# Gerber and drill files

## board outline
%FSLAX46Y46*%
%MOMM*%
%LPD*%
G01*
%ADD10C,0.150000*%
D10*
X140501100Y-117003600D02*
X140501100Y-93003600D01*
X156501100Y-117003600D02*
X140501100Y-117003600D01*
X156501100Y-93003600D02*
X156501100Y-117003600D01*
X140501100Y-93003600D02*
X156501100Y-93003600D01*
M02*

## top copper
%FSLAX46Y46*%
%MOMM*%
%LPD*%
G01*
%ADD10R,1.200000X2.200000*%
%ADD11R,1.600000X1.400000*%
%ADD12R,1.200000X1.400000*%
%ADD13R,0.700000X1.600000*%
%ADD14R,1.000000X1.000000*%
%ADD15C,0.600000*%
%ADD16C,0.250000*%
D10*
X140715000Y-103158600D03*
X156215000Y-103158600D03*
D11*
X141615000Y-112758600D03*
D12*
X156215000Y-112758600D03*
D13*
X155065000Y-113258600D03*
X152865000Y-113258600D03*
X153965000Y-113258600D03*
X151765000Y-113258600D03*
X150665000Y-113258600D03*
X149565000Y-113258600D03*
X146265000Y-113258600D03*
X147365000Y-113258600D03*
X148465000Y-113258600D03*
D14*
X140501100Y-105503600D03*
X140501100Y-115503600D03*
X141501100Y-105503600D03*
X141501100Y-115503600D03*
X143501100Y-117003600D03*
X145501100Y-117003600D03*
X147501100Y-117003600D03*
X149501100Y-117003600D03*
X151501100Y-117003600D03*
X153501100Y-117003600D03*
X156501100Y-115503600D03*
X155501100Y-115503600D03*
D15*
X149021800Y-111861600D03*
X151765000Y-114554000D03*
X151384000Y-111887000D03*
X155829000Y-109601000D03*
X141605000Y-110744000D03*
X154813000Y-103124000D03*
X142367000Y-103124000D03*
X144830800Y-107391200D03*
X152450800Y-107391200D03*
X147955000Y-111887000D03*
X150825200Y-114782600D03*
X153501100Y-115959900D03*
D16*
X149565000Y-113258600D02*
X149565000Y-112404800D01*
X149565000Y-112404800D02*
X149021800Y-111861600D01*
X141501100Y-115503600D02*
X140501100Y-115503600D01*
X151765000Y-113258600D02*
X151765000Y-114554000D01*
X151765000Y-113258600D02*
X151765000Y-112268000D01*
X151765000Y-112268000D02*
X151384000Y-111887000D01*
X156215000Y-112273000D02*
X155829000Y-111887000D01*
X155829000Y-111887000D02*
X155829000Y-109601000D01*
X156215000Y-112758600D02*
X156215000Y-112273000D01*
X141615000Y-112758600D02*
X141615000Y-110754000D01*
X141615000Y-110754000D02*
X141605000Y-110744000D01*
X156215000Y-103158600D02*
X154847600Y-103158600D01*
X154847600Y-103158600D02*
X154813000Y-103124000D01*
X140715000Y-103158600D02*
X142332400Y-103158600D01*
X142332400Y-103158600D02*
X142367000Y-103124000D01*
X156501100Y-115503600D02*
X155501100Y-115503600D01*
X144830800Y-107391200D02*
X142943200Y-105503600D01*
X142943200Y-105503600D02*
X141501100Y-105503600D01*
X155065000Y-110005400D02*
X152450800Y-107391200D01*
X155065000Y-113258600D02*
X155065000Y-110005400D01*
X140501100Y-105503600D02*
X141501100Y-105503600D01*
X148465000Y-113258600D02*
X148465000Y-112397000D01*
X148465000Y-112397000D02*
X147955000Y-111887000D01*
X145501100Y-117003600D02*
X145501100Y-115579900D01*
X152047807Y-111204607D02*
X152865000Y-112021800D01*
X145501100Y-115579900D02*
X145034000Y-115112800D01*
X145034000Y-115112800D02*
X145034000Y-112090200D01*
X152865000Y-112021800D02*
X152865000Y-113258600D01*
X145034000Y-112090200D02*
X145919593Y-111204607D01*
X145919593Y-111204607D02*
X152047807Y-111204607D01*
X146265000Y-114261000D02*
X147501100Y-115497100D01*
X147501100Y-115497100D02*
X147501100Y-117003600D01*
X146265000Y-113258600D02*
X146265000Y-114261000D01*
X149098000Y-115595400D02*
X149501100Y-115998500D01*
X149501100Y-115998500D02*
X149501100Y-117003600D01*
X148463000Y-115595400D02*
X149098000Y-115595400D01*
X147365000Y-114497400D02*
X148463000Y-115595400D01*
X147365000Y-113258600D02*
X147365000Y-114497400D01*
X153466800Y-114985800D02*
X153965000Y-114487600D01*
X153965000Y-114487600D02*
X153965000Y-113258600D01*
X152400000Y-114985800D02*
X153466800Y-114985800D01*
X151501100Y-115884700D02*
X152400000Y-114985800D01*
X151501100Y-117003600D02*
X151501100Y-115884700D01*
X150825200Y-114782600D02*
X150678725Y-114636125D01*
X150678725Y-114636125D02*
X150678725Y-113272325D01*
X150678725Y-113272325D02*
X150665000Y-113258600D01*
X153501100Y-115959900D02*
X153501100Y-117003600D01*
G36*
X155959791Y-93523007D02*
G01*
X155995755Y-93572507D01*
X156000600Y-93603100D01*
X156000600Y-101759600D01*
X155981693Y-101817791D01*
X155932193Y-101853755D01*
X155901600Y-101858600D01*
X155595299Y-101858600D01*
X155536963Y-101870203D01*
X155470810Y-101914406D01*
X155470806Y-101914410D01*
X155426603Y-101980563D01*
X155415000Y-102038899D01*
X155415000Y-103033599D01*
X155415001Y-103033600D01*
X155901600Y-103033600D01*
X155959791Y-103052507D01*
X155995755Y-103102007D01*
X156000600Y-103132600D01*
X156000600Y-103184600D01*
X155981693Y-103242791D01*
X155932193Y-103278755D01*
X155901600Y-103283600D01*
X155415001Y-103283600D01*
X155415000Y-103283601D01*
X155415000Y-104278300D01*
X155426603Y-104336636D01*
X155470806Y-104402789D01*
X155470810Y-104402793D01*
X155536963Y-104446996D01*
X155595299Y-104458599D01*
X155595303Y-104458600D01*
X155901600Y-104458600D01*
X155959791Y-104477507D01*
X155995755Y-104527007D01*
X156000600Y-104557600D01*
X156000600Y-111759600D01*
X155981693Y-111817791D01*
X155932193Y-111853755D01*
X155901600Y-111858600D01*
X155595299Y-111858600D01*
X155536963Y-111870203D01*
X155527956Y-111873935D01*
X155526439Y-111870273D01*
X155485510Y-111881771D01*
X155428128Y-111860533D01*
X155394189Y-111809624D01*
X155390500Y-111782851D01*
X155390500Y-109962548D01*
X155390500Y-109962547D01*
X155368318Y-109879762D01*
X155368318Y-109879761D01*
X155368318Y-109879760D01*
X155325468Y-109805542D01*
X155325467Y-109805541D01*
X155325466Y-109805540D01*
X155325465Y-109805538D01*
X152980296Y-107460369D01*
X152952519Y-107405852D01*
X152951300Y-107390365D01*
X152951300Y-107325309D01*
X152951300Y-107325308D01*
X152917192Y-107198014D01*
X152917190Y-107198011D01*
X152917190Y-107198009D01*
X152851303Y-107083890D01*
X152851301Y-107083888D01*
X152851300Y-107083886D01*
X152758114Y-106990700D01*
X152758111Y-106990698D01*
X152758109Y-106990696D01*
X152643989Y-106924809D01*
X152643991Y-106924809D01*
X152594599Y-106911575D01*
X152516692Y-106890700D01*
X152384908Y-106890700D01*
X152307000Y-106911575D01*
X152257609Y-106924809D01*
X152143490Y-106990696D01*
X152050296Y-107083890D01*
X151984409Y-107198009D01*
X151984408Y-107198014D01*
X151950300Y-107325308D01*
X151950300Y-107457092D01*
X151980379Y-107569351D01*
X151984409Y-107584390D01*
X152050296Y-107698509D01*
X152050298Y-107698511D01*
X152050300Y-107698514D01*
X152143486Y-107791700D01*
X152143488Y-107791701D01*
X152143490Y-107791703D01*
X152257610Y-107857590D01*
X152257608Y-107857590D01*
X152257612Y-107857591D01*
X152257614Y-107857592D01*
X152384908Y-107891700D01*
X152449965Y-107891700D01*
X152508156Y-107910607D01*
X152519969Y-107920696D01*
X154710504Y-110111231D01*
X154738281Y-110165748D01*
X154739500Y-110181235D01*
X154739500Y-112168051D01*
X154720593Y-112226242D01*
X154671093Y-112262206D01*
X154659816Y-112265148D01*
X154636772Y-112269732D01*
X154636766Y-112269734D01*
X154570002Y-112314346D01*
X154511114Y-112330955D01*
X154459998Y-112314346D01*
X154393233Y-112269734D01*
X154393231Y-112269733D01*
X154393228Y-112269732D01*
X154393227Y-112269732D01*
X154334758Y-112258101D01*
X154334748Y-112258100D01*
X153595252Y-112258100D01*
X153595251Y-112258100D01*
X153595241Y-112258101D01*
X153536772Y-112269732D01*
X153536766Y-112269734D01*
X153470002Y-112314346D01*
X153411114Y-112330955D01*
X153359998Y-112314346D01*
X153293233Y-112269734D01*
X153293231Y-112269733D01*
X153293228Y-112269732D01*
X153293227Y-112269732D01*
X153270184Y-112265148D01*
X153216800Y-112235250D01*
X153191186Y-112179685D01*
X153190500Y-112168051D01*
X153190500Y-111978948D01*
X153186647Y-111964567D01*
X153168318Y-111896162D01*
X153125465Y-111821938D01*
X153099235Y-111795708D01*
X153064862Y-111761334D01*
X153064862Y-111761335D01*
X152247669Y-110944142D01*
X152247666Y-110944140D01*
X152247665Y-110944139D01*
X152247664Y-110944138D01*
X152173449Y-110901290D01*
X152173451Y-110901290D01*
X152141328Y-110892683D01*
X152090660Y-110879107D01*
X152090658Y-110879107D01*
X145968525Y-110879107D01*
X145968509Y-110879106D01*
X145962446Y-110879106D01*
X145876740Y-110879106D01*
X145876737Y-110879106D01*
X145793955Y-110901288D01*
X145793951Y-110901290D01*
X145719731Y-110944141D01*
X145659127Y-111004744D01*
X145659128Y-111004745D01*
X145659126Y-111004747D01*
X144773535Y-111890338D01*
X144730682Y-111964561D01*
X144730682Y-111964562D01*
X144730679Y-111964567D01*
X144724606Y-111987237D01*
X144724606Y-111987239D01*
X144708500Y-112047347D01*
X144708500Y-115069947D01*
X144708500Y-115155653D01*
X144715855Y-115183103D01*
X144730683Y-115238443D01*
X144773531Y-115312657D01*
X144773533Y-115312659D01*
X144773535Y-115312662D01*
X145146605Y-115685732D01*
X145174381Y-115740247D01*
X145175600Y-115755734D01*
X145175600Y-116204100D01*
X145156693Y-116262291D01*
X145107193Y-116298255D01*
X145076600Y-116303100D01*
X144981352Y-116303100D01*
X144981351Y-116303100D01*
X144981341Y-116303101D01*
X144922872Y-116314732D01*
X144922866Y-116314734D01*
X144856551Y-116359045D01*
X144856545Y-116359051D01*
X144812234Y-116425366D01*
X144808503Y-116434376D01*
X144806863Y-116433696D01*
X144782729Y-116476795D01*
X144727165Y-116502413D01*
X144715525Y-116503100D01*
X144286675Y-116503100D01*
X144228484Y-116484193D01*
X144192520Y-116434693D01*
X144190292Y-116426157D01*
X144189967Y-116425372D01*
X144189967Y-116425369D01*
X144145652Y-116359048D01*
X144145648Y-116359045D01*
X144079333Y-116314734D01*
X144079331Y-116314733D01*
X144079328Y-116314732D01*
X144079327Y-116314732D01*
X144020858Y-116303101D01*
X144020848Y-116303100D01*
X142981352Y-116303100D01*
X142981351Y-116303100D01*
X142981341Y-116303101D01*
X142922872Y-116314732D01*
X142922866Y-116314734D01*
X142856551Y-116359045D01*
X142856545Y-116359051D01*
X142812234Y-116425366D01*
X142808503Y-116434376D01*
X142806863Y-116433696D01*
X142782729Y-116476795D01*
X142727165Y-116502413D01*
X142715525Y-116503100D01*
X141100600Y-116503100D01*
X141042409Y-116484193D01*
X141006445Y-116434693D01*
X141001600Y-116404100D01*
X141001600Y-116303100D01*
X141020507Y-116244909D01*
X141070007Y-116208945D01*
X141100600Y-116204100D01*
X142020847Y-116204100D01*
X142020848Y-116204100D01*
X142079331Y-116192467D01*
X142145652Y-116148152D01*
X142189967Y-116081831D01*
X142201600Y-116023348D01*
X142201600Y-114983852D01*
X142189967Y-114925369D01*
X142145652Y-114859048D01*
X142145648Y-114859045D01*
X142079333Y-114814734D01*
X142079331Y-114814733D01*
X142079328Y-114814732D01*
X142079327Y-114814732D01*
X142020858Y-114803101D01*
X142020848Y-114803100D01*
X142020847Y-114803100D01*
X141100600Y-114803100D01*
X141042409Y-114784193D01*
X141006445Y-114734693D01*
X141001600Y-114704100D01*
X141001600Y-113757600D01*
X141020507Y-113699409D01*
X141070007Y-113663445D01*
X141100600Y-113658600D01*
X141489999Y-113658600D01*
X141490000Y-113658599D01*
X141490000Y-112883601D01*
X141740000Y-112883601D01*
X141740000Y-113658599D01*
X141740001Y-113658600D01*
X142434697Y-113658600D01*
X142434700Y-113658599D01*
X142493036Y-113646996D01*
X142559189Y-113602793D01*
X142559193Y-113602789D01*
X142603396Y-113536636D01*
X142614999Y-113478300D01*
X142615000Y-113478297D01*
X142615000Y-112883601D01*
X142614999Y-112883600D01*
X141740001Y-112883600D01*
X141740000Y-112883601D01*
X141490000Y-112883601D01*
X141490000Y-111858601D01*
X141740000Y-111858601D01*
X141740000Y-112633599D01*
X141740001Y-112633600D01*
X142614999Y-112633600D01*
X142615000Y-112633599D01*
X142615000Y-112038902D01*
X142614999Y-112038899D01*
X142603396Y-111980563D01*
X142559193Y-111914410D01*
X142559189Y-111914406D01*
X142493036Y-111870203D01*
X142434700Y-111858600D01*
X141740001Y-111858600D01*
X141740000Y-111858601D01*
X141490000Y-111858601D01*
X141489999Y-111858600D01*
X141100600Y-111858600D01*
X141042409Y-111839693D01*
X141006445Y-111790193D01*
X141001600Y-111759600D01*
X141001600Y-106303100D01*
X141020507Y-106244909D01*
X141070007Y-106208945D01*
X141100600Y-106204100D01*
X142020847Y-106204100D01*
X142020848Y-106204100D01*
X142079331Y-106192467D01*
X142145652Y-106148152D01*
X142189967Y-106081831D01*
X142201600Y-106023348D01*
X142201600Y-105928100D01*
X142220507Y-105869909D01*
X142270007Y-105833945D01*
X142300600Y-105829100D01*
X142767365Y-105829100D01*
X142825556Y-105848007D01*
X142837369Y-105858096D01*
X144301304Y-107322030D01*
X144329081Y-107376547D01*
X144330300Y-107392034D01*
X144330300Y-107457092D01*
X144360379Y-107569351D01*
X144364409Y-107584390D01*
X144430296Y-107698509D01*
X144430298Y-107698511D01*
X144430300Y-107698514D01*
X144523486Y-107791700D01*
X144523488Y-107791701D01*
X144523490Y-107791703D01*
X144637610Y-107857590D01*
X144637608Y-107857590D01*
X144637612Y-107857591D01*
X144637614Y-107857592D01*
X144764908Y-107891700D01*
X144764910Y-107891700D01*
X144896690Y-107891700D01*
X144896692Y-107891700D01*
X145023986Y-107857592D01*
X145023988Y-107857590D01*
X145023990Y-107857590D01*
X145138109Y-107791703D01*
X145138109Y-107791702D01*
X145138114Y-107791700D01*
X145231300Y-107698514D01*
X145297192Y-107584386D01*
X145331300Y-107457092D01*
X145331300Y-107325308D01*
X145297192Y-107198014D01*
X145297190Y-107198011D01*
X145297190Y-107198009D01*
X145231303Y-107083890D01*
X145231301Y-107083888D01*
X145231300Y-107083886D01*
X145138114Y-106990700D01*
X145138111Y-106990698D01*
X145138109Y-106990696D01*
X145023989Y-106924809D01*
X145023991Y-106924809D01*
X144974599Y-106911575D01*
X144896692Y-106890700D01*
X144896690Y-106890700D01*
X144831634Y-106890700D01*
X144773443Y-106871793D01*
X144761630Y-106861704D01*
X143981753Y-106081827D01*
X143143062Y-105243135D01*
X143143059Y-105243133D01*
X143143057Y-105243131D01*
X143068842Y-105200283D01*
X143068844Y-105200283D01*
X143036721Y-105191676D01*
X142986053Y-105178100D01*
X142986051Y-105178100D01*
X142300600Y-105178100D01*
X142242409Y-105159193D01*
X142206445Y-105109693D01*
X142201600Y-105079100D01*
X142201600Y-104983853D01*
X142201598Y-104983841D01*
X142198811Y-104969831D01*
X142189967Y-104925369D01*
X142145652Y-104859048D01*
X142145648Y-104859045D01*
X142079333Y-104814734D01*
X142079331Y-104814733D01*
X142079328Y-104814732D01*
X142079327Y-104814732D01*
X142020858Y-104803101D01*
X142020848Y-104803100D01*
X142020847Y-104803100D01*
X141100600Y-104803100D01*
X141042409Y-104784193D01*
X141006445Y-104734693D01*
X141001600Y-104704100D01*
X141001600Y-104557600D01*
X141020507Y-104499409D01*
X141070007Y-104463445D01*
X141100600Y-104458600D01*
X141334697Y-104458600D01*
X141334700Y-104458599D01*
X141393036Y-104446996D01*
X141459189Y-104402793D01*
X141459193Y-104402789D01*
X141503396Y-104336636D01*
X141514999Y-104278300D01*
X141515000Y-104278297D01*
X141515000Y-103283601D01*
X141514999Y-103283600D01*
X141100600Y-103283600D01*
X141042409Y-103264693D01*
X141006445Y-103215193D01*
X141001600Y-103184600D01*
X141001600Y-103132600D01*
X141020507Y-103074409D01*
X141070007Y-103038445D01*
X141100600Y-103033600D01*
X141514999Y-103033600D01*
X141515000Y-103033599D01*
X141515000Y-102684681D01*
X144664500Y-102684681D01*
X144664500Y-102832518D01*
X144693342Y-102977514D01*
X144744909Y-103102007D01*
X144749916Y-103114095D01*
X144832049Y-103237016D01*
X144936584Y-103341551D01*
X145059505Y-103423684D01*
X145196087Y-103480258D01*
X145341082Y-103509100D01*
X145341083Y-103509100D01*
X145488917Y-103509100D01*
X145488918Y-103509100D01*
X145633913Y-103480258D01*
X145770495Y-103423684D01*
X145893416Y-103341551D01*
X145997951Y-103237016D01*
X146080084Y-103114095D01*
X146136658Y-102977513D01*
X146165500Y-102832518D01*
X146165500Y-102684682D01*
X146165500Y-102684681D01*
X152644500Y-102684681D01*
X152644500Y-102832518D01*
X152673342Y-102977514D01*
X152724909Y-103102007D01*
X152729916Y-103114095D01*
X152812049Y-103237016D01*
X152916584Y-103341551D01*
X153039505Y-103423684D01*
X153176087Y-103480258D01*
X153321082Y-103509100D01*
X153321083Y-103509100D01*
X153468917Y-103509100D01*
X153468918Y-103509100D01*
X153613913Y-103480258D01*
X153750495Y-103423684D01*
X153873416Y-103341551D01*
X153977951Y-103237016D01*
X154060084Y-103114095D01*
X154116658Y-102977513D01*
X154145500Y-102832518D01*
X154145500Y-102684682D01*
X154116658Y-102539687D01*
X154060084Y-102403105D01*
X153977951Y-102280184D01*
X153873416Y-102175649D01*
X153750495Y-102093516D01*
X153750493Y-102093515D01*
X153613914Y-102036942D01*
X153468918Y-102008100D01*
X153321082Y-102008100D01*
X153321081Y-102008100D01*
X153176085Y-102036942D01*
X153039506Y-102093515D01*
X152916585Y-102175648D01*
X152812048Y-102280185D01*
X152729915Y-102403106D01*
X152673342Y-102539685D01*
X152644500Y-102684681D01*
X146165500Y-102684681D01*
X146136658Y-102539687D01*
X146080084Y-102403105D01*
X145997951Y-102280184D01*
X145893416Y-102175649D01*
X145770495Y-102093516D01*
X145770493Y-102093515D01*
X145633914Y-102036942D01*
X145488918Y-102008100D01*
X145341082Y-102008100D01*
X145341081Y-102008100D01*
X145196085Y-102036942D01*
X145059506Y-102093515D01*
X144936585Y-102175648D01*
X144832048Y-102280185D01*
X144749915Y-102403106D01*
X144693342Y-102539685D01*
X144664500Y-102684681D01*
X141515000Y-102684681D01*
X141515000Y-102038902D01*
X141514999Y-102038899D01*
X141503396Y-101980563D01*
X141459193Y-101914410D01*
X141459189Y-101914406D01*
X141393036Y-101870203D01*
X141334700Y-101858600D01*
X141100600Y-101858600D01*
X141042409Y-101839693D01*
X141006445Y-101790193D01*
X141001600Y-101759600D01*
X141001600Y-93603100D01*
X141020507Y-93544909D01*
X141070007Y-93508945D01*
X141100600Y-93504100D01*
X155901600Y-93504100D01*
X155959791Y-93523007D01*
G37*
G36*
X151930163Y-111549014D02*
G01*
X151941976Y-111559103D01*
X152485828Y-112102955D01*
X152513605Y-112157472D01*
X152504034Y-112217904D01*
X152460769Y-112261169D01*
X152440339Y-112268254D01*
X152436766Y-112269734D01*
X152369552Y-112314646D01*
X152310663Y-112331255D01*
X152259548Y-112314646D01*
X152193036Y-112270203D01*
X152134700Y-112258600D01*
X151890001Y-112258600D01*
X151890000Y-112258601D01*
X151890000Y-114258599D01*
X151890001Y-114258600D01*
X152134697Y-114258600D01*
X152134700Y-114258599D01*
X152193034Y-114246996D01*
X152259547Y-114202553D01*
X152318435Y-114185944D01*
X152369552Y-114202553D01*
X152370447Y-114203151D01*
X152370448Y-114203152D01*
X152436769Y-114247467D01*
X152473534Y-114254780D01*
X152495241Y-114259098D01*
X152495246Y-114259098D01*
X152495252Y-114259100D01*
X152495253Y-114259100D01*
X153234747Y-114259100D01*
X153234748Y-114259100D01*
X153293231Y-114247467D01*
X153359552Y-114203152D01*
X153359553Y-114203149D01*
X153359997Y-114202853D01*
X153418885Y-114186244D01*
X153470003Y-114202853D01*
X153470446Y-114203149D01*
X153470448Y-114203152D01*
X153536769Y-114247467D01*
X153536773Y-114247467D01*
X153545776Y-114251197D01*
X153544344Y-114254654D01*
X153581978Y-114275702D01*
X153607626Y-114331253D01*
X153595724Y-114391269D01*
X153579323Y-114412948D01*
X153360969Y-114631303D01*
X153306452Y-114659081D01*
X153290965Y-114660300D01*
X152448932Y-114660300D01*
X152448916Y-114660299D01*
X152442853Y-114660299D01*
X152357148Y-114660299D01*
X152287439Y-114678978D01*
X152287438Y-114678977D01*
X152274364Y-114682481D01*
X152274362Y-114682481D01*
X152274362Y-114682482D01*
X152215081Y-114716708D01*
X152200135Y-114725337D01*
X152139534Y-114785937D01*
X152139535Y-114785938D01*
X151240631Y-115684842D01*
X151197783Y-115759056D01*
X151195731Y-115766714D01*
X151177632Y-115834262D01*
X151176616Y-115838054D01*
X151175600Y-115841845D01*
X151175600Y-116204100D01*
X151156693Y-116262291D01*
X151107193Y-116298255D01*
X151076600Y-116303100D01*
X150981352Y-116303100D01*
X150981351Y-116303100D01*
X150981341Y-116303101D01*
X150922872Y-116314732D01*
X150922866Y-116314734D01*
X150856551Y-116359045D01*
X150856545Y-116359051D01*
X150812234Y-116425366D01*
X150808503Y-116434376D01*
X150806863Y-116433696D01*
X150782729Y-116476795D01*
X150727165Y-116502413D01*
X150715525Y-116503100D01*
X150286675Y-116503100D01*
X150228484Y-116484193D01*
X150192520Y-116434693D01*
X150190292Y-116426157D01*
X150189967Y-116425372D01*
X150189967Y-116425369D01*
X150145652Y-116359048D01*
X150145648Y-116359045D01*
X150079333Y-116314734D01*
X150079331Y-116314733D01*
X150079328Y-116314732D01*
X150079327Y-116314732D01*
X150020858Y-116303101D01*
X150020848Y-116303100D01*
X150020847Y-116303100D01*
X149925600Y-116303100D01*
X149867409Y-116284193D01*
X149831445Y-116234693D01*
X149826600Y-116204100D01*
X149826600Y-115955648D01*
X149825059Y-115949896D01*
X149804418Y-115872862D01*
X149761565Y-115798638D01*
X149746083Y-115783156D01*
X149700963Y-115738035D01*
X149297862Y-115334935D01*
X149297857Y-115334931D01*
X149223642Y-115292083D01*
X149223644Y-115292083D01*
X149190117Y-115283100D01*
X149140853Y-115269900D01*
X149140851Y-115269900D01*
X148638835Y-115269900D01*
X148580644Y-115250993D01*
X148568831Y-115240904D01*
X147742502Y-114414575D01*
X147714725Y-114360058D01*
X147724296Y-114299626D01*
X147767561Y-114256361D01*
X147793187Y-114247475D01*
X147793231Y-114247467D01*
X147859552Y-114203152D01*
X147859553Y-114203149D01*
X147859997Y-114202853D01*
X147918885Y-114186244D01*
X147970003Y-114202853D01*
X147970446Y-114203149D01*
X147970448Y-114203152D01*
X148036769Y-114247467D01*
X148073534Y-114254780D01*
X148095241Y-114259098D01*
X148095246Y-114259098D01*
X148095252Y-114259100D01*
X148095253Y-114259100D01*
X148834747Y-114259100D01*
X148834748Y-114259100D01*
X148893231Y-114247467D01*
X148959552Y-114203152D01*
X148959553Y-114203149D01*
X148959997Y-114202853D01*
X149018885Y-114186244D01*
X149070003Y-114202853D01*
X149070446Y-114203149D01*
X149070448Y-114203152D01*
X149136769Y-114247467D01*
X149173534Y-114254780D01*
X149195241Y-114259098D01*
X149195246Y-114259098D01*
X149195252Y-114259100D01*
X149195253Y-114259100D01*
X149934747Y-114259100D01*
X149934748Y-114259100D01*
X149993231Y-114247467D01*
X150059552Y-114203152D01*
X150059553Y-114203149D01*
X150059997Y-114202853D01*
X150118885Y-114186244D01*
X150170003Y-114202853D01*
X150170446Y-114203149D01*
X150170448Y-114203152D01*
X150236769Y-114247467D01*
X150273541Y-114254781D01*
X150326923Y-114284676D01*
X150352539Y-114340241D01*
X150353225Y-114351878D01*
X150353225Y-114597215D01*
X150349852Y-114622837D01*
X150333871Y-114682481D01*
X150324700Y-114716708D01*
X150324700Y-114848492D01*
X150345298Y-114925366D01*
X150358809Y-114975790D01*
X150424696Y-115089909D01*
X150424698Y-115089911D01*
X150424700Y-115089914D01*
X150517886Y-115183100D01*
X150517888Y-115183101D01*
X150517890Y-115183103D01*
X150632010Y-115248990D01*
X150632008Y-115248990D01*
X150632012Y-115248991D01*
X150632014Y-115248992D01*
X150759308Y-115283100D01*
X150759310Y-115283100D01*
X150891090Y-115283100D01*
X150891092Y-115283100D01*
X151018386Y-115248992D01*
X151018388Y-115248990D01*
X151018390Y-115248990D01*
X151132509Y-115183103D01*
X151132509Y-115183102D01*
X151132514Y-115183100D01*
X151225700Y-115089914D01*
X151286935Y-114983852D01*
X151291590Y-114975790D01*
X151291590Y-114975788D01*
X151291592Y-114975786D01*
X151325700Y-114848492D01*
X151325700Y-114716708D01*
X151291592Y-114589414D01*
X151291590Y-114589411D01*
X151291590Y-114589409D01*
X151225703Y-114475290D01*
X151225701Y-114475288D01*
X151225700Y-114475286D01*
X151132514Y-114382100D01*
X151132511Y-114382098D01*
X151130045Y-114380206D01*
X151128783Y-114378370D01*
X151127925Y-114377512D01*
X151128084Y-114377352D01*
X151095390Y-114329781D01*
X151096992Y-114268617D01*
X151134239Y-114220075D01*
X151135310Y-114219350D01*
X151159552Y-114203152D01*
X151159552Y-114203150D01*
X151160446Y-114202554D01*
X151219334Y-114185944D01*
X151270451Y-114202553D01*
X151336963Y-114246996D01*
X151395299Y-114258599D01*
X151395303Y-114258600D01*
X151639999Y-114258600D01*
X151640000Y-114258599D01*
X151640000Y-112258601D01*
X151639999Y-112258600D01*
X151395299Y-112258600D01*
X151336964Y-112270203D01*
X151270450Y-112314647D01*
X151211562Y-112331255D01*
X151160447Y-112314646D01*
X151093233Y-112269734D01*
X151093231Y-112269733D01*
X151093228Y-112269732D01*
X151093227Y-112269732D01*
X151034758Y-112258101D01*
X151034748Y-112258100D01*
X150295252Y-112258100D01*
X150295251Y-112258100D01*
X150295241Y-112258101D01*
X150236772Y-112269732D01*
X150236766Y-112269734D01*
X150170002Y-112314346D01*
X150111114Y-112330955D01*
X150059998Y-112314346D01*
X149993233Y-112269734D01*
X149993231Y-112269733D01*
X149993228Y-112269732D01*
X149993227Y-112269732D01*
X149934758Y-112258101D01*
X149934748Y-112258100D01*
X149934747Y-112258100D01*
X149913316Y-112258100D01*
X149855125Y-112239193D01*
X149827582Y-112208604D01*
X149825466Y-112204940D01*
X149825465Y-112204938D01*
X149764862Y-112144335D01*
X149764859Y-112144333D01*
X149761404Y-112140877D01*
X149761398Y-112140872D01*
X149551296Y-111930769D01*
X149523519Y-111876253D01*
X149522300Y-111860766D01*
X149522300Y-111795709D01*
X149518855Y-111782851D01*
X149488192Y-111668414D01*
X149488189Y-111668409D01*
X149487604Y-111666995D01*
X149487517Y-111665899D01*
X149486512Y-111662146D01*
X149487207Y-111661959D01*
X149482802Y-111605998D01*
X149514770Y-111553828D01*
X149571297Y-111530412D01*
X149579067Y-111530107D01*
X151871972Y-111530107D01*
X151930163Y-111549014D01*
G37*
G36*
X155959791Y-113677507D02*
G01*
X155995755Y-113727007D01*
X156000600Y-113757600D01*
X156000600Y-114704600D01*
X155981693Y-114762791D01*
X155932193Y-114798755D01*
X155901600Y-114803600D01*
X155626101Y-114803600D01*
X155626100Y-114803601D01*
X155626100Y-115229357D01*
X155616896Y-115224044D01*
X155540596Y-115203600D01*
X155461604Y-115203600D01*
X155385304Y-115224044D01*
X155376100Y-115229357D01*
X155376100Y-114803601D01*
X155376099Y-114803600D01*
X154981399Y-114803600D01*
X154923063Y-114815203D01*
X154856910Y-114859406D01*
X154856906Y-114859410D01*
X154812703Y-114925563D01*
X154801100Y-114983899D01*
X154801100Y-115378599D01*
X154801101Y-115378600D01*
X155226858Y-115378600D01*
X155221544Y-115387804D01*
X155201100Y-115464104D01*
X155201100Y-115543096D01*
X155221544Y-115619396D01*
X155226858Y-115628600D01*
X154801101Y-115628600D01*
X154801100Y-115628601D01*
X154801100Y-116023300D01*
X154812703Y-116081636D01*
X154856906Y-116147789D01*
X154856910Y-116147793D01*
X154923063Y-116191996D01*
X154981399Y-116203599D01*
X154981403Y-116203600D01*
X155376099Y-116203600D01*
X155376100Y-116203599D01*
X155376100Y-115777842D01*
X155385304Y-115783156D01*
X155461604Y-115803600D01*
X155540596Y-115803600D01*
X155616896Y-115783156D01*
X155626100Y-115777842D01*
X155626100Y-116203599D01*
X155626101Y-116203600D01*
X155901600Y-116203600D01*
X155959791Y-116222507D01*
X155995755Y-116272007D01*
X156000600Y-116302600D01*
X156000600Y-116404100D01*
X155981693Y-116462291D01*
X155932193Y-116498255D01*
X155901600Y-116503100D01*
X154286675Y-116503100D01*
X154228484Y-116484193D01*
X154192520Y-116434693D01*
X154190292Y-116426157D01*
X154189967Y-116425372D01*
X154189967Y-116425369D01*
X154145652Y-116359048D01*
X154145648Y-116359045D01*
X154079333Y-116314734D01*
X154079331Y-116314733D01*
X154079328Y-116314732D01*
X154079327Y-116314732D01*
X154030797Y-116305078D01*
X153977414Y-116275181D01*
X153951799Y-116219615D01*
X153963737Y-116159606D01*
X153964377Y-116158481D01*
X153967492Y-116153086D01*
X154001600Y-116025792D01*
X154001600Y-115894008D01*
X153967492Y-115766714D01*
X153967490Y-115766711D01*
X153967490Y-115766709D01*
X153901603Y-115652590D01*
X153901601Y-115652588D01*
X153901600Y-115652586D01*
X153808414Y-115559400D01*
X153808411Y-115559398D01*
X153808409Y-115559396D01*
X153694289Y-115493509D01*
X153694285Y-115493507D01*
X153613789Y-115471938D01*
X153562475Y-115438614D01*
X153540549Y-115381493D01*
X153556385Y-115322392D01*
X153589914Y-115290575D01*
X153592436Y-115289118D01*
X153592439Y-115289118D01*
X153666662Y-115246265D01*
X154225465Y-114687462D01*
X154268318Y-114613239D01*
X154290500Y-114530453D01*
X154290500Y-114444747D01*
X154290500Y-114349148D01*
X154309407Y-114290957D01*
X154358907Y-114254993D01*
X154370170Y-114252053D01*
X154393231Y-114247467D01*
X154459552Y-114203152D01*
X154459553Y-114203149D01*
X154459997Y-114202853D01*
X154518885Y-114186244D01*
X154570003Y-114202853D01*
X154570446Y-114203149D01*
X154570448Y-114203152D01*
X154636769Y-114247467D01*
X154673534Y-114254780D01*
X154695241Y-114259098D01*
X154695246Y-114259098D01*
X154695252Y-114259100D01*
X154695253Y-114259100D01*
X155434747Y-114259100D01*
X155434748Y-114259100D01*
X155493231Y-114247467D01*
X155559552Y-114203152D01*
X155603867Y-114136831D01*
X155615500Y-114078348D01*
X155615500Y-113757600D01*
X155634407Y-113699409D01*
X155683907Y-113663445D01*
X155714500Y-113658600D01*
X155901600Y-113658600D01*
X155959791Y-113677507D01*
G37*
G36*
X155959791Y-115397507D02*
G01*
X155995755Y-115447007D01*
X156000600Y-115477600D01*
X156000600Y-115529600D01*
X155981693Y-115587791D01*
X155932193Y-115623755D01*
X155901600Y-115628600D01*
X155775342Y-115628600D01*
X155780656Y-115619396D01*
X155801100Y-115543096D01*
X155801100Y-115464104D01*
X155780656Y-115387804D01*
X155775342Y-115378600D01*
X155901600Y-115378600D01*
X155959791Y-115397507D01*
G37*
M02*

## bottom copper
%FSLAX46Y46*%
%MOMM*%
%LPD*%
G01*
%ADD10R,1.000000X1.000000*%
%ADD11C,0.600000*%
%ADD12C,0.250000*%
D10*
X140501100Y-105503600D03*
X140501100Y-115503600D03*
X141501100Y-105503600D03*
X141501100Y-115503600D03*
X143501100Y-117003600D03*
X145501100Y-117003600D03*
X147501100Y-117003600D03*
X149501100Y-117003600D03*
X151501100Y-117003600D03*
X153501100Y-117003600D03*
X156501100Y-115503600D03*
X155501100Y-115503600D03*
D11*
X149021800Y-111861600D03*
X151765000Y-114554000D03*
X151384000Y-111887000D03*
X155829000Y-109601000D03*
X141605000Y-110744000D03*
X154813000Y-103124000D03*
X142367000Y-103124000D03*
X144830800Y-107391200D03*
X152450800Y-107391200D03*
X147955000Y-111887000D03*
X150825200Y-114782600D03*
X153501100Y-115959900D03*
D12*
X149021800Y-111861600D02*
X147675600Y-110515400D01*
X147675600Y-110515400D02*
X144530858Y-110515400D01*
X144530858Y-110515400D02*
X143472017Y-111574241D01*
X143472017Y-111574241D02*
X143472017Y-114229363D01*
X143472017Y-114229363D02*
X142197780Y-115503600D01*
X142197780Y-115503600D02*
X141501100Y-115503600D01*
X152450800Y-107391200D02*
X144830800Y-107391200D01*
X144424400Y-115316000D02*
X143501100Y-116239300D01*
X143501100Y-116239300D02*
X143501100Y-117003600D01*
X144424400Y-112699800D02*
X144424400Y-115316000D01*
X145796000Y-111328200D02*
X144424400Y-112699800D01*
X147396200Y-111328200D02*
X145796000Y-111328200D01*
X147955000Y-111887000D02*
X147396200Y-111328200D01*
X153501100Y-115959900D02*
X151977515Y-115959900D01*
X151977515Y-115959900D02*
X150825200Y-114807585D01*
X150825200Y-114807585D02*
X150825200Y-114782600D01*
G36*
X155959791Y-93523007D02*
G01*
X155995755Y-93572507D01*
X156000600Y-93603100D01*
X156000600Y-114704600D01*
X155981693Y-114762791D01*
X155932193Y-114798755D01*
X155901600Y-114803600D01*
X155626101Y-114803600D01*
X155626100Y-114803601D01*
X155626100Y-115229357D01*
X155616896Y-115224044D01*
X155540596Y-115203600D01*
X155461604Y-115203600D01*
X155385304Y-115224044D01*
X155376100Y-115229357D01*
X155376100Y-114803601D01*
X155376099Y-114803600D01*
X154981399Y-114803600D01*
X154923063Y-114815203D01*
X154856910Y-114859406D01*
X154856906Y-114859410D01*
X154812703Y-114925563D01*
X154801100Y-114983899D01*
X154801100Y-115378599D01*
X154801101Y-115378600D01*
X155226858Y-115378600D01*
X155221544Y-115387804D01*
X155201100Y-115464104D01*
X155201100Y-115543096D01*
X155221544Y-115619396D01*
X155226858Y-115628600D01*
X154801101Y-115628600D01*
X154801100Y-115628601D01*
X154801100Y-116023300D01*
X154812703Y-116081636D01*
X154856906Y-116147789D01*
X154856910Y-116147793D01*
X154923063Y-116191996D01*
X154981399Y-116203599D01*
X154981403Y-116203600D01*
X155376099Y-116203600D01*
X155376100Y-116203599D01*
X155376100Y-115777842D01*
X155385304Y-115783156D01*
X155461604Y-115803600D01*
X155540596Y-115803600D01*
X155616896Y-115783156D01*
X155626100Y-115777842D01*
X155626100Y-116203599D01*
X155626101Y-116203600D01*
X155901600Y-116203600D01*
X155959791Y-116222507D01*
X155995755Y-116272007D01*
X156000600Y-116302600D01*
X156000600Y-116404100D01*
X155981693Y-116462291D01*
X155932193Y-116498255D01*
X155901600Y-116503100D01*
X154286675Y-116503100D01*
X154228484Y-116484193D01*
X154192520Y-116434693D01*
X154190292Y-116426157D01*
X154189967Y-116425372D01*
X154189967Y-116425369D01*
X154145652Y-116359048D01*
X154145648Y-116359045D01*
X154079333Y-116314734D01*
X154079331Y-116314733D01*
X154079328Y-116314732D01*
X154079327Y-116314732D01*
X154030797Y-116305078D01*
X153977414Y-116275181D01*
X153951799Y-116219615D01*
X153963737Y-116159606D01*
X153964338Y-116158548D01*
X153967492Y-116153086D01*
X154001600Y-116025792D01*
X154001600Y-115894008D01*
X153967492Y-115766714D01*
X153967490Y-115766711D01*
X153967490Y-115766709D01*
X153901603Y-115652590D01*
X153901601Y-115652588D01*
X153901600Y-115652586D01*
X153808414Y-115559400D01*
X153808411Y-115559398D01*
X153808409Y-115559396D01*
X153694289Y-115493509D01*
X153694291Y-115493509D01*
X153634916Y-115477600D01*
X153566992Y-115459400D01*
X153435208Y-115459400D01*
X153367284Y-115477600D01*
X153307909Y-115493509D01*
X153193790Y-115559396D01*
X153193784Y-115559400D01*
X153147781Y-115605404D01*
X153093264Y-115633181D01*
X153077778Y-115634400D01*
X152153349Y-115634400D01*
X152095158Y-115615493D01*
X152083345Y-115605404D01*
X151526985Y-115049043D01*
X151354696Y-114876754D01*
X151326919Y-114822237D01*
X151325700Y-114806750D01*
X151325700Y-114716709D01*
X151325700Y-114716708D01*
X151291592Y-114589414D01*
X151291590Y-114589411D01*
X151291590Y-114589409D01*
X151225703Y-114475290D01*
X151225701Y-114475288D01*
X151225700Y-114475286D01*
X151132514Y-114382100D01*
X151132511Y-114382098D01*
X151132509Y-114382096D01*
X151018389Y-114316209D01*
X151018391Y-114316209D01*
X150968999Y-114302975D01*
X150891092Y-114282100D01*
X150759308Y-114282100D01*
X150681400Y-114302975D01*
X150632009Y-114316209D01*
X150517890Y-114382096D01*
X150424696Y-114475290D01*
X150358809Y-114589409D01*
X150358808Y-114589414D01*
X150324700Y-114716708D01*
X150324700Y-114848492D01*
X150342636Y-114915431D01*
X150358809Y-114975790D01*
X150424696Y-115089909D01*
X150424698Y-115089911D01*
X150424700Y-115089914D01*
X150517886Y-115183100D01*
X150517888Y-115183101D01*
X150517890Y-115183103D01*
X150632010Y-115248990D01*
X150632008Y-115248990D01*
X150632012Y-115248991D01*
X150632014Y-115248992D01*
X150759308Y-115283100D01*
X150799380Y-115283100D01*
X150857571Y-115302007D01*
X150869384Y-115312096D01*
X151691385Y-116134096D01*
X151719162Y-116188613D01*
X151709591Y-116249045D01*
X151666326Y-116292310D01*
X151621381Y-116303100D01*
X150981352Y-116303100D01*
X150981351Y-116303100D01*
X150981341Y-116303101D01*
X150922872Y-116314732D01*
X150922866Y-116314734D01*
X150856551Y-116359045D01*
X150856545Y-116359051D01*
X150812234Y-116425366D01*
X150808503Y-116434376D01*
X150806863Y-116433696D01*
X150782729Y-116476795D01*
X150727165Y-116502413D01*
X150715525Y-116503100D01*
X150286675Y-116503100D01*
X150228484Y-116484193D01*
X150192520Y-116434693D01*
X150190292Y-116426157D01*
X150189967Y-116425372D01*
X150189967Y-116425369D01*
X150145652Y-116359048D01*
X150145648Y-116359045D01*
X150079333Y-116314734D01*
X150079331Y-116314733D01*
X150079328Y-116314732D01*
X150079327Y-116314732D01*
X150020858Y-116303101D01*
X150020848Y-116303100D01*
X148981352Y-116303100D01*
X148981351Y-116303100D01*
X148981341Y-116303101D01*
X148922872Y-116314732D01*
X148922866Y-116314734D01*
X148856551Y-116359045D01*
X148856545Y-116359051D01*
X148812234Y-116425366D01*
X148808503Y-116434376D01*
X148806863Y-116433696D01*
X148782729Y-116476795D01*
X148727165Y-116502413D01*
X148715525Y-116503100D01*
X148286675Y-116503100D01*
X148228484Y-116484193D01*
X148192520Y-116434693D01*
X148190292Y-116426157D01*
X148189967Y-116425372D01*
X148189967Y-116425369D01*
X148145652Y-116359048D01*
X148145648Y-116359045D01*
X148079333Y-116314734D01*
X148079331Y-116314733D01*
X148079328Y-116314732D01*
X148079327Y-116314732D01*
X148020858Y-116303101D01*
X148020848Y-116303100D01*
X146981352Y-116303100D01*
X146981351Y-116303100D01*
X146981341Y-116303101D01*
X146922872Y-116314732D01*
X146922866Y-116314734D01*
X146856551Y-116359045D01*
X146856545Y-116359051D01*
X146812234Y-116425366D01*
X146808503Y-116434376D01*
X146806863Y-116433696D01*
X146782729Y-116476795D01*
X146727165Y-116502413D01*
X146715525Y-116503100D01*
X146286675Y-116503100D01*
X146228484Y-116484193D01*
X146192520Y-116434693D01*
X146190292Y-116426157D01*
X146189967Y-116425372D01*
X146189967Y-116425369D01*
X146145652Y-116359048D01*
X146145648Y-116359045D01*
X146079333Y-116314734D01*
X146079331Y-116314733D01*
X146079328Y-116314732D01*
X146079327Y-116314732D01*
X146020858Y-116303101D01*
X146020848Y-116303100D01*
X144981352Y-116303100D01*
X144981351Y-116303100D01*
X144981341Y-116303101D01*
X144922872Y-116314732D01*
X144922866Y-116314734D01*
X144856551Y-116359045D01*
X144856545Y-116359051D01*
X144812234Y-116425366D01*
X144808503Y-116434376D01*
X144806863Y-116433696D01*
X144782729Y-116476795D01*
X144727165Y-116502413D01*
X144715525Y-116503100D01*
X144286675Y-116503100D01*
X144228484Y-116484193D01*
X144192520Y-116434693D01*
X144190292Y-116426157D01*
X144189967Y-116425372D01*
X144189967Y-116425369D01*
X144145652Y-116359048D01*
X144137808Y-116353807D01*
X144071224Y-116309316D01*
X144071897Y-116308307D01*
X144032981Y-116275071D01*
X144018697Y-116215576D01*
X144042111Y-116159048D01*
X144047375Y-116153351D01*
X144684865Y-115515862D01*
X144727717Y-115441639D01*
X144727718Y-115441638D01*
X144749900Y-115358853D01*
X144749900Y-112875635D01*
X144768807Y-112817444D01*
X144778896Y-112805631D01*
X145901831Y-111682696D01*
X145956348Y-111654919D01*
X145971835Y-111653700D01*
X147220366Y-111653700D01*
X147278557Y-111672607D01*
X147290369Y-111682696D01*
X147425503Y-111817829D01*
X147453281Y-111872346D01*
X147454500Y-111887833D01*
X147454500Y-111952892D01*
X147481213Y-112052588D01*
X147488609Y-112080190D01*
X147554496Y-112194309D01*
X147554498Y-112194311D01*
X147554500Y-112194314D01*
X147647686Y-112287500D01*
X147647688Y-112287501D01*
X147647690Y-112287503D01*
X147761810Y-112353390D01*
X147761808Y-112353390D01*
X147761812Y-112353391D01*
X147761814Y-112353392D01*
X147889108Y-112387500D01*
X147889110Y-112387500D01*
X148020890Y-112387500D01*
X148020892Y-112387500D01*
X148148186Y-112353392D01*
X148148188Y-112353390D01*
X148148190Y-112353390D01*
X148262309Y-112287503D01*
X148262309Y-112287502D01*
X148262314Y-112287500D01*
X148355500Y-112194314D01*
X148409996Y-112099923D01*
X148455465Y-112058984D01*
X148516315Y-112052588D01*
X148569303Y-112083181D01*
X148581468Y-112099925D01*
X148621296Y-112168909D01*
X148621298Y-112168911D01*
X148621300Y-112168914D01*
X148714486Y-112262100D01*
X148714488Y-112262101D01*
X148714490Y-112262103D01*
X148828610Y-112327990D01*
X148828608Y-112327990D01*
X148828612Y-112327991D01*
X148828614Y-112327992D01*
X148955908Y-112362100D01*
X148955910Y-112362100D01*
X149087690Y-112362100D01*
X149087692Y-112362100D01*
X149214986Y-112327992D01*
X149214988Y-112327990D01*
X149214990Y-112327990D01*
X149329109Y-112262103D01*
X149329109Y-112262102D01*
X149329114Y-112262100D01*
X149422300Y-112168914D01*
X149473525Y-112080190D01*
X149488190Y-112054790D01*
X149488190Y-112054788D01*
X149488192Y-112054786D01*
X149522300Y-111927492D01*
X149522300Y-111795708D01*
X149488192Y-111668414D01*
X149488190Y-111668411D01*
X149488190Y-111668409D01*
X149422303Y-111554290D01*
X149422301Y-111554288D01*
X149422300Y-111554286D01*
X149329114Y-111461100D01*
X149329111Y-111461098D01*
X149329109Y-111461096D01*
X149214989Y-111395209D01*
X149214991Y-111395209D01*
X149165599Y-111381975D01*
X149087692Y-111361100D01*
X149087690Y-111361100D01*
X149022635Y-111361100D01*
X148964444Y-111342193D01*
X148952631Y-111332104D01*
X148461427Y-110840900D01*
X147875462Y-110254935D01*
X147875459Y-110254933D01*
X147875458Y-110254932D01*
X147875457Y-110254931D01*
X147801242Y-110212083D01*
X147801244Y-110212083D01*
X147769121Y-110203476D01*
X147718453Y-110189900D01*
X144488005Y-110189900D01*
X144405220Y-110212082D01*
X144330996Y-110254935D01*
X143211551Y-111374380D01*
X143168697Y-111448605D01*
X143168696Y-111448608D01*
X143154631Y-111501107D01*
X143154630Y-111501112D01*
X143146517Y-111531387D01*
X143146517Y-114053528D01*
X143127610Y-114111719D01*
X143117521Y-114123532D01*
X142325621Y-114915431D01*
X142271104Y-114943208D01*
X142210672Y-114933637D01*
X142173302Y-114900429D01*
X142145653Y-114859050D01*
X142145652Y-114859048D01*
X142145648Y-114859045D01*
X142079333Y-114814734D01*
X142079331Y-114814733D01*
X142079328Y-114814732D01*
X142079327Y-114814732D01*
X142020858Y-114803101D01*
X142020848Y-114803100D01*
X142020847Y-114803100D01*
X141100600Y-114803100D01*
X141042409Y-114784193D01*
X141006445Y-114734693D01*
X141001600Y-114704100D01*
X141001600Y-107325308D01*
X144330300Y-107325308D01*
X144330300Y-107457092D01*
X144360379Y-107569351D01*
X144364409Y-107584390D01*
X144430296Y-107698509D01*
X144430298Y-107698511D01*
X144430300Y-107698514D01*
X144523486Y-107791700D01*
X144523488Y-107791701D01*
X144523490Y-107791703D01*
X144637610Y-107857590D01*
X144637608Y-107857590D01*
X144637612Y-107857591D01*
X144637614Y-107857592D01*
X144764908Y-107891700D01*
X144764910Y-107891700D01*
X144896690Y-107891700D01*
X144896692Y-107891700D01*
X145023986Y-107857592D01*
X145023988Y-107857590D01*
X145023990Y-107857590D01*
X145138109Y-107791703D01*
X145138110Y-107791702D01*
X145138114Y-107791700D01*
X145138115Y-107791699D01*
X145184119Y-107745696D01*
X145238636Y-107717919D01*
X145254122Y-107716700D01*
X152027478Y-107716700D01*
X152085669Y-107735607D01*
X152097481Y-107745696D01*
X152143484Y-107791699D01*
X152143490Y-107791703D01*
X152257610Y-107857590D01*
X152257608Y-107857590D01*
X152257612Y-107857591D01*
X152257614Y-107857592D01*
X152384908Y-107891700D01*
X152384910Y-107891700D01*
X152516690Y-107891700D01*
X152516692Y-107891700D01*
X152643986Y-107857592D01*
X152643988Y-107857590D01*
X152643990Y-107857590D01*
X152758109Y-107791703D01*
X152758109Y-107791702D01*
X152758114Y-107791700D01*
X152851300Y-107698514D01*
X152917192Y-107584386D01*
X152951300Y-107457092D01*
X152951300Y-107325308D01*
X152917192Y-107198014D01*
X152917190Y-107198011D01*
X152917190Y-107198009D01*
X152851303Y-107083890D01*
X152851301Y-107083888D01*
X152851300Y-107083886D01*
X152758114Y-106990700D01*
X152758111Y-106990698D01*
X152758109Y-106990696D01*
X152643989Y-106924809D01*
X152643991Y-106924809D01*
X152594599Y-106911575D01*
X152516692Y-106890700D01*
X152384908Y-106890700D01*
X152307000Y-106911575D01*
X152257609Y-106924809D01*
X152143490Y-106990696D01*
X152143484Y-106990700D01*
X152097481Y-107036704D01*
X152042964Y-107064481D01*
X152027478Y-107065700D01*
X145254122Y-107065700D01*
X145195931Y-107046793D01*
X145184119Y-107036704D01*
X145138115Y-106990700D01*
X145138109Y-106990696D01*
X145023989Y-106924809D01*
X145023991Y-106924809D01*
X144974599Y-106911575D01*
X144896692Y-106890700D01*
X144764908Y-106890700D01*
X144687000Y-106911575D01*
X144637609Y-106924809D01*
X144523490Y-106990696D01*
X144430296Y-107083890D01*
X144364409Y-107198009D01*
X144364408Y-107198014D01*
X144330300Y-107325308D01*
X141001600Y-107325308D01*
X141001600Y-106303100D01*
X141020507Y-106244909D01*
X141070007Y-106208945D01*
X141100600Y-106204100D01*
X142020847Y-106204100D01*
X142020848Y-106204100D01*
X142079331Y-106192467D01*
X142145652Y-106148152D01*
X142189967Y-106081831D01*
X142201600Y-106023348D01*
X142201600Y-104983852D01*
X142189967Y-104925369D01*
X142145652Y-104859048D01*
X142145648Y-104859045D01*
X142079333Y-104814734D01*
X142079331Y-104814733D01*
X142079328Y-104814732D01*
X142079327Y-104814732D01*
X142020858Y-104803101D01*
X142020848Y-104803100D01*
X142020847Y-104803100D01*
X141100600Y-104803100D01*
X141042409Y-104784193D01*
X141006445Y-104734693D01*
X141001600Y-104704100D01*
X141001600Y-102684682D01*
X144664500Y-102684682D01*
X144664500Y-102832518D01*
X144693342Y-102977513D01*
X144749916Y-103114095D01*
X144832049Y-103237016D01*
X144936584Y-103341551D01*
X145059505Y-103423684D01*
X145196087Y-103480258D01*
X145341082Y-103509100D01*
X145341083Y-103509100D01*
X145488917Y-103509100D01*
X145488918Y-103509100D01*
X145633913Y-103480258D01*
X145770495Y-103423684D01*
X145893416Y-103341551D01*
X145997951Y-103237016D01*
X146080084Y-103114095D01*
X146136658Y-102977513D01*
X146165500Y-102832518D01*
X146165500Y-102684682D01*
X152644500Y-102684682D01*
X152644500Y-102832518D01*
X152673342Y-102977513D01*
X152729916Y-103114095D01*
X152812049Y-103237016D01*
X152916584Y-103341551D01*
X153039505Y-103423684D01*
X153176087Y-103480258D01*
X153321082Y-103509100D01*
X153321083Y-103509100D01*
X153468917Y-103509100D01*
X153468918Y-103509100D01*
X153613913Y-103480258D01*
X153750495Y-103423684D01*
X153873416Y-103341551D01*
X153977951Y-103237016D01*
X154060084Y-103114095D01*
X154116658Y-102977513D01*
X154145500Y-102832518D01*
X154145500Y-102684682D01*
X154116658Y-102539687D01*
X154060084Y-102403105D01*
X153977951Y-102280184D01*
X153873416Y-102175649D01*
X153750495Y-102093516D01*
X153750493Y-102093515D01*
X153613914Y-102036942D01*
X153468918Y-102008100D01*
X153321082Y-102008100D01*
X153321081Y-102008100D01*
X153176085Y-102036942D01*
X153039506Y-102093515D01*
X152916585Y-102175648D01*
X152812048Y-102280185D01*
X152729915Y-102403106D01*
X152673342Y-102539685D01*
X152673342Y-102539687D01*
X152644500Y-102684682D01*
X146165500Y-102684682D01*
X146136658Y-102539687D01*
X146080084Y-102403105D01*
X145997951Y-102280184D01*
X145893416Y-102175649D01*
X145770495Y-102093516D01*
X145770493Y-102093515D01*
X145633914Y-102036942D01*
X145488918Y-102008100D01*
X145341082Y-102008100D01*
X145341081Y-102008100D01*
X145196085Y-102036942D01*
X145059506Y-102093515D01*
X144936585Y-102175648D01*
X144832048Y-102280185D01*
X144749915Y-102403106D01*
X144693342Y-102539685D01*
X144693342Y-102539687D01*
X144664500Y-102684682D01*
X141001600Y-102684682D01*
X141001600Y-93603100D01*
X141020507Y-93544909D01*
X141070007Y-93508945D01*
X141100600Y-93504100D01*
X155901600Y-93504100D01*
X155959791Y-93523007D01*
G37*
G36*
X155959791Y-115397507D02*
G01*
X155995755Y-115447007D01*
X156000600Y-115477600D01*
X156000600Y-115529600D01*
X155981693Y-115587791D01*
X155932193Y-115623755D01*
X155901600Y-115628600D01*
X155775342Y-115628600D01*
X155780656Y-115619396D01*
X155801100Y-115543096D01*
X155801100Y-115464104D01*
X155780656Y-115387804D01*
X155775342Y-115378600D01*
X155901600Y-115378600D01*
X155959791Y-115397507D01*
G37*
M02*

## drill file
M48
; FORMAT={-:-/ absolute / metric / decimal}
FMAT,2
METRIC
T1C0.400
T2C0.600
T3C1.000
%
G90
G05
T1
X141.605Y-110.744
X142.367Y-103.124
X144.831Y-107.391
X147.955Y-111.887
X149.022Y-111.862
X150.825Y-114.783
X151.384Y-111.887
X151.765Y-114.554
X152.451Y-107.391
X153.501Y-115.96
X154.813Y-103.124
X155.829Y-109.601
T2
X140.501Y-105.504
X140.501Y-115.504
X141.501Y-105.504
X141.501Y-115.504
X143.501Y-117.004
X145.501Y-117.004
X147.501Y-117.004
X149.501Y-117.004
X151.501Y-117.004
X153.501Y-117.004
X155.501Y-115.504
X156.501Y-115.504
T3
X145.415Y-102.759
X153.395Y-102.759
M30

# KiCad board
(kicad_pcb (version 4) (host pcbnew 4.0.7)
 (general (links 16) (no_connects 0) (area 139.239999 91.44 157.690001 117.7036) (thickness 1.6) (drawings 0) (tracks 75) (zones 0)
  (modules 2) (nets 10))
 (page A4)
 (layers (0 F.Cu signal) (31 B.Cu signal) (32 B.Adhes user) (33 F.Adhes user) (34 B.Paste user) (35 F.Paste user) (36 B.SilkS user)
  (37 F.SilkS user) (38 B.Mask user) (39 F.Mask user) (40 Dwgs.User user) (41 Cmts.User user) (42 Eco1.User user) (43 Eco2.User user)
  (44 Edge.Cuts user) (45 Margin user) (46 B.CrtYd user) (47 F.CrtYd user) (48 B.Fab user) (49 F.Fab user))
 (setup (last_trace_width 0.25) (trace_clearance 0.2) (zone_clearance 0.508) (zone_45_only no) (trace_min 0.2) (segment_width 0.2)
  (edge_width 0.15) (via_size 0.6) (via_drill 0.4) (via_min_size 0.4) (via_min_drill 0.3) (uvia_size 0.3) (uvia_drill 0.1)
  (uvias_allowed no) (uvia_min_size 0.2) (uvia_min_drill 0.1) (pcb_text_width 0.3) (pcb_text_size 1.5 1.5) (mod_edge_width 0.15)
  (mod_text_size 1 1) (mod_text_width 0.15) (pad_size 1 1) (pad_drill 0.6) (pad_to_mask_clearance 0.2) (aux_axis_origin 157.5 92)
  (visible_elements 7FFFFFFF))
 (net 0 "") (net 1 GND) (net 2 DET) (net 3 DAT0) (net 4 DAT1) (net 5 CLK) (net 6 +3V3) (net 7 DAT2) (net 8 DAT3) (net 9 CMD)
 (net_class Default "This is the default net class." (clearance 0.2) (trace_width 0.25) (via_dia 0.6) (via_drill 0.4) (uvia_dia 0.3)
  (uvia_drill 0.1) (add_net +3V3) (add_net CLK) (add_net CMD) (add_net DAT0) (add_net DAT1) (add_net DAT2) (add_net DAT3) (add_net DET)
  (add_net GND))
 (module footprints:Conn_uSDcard (layer F.Cu) (at 148.465 102.7586 180)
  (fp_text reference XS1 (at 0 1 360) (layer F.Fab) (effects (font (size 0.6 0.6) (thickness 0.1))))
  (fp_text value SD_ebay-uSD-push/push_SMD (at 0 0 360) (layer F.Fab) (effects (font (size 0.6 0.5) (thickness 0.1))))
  (pad 6 smd rect (at 7.75 -0.4 180) (size 1.2 2.2) (layers F.Cu F.Paste F.Mask) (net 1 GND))
  (pad 6 smd rect (at -7.75 -0.4 180) (size 1.2 2.2) (layers F.Cu F.Paste F.Mask) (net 1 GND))
  (pad 6 smd rect (at 6.85 -10 180) (size 1.6 1.4) (layers F.Cu F.Paste F.Mask) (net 1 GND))
  (pad 6 smd rect (at -7.75 -10 180) (size 1.2 1.4) (layers F.Cu F.Paste F.Mask) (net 1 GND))
  (pad 9 smd rect (at -6.6 -10.5 180) (size 0.7 1.6) (layers F.Cu F.Paste F.Mask) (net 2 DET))
  (pad 7 smd rect (at -4.4 -10.5 180) (size 0.7 1.6) (layers F.Cu F.Paste F.Mask) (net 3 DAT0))
  (pad 8 smd rect (at -5.5 -10.5 180) (size 0.7 1.6) (layers F.Cu F.Paste F.Mask) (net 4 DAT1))
  (pad 6 smd rect (at -3.3 -10.5 180) (size 0.7 1.6) (layers F.Cu F.Paste F.Mask) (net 1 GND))
  (pad 5 smd rect (at -2.2 -10.5 180) (size 0.7 1.6) (layers F.Cu F.Paste F.Mask) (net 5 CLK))
  (pad 4 smd rect (at -1.1 -10.5 180) (size 0.7 1.6) (layers F.Cu F.Paste F.Mask) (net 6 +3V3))
  (pad 1 smd rect (at 2.2 -10.5 180) (size 0.7 1.6) (layers F.Cu F.Paste F.Mask) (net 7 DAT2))
  (pad 2 smd rect (at 1.1 -10.5 180) (size 0.7 1.6) (layers F.Cu F.Paste F.Mask) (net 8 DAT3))
  (pad "" np_thru_hole circle (at 3.05 0 180) (size 1 1) (drill 1) (layers *.Cu))
  (pad "" np_thru_hole circle (at -4.93 0 180) (size 1 1) (drill 1) (layers *.Cu))
  (pad 3 smd rect (at 0 -10.5 180) (size 0.7 1.6) (layers F.Cu F.Paste F.Mask) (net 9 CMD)))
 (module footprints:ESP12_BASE (layer F.Cu) (at 148.5011 105.0036)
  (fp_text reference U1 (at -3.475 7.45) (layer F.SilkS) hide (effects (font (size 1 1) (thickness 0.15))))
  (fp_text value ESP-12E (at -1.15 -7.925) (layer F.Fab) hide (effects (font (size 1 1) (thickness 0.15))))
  (fp_line (start -8 12) (end -8 -12) (layer Edge.Cuts) (width 0.15))
  (fp_line (start 8 12) (end -8 12) (layer Edge.Cuts) (width 0.15))
  (fp_line (start 8 -12) (end 8 12) (layer Edge.Cuts) (width 0.15))
  (fp_line (start -8 -12) (end 8 -12) (layer Edge.Cuts) (width 0.15))
  (pad 3 thru_hole rect (at -8 0.5) (size 1 1) (drill 0.6) (layers *.Cu B.Mask) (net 2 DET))
  (pad 8 thru_hole rect (at -8 10.5) (size 1 1) (drill 0.6) (layers *.Cu *.Mask) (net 6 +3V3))
  (pad 3 thru_hole rect (at -7 0.5) (size 1 1) (drill 0.6) (layers *.Cu B.Mask) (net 2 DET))
  (pad 8 thru_hole rect (at -7 10.5) (size 1 1) (drill 0.6) (layers *.Cu *.Mask) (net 6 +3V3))
  (pad 9 thru_hole rect (at -5 12) (size 1 1) (drill 0.6) (layers *.Cu *.Mask) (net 9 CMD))
  (pad 10 thru_hole rect (at -3 12) (size 1 1) (drill 0.6) (layers *.Cu *.Mask) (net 3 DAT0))
  (pad 11 thru_hole rect (at -1 12) (size 1 1) (drill 0.6) (layers *.Cu *.Mask) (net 7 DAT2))
  (pad 12 thru_hole rect (at 1 12) (size 1 1) (drill 0.6) (layers *.Cu *.Mask) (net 8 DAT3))
  (pad 13 thru_hole rect (at 3 12) (size 1 1) (drill 0.6) (layers *.Cu *.Mask) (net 4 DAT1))
  (pad 14 thru_hole rect (at 5 12) (size 1 1) (drill 0.6) (layers *.Cu *.Mask) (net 5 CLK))
  (pad 15 thru_hole rect (at 8 10.5) (size 1 1) (drill 0.6) (layers *.Cu *.Mask) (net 1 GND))
  (pad 15 thru_hole rect (at 7 10.5) (size 1 1) (drill 0.6) (layers *.Cu *.Mask) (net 1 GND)))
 (segment (start 149.0218 111.8616) (end 147.6756 110.5154) (width 0.25) (layer B.Cu) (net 6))
 (segment (start 147.6756 110.5154) (end 144.530858 110.5154) (width 0.25) (layer B.Cu) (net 6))
 (segment (start 144.530858 110.5154) (end 143.472017 111.574241) (width 0.25) (layer B.Cu) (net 6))
 (segment (start 143.472017 111.574241) (end 143.472017 114.229363) (width 0.25) (layer B.Cu) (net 6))
 (segment (start 143.472017 114.229363) (end 142.19778 115.5036) (width 0.25) (layer B.Cu) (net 6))
 (segment (start 142.19778 115.5036) (end 141.5011 115.5036) (width 0.25) (layer B.Cu) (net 6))
 (segment (start 149.565 113.2586) (end 149.565 112.4048) (width 0.25) (layer F.Cu) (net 6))
 (segment (start 149.565 112.4048) (end 149.0218 111.8616) (width 0.25) (layer F.Cu) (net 6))
 (via (at 149.0218 111.8616) (size 0.6) (drill 0.4) (layers F.Cu B.Cu) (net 6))
 (segment (start 141.5011 115.5036) (end 140.5011 115.5036) (width 0.25) (layer F.Cu) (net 6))
 (segment (start 151.765 113.2586) (end 151.765 114.554) (width 0.25) (layer F.Cu) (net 1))
 (via (at 151.765 114.554) (size 0.6) (drill 0.4) (layers F.Cu B.Cu) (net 1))
 (segment (start 151.765 113.2586) (end 151.765 112.268) (width 0.25) (layer F.Cu) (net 1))
 (via (at 151.384 111.887) (size 0.6) (drill 0.4) (layers F.Cu B.Cu) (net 1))
 (segment (start 151.765 112.268) (end 151.384 111.887) (width 0.25) (layer F.Cu) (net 1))
 (segment (start 156.215 112.273) (end 155.829 111.887) (width 0.25) (layer F.Cu) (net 1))
 (segment (start 155.829 111.887) (end 155.829 109.601) (width 0.25) (layer F.Cu) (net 1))
 (via (at 155.829 109.601) (size 0.6) (drill 0.4) (layers F.Cu B.Cu) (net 1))
 (segment (start 156.215 112.7586) (end 156.215 112.273) (width 0.25) (layer F.Cu) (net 1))
 (segment (start 141.615 112.7586) (end 141.615 110.754) (width 0.25) (layer F.Cu) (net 1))
 (segment (start 141.615 110.754) (end 141.605 110.744) (width 0.25) (layer F.Cu) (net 1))
 (via (at 141.605 110.744) (size 0.6) (drill 0.4) (layers F.Cu B.Cu) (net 1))
 (segment (start 156.215 103.1586) (end 154.8476 103.1586) (width 0.25) (layer F.Cu) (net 1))
 (segment (start 154.8476 103.1586) (end 154.813 103.124) (width 0.25) (layer F.Cu) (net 1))
 (via (at 154.813 103.124) (size 0.6) (drill 0.4) (layers F.Cu B.Cu) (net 1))
 (segment (start 140.715 103.1586) (end 142.3324 103.1586) (width 0.25) (layer F.Cu) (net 1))
 (segment (start 142.3324 103.1586) (end 142.367 103.124) (width 0.25) (layer F.Cu) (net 1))
 (via (at 142.367 103.124) (size 0.6) (drill 0.4) (layers F.Cu B.Cu) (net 1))
 (segment (start 156.5011 115.5036) (end 155.5011 115.5036) (width 0.25) (layer F.Cu) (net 1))
 (segment (start 152.4508 107.3912) (end 144.8308 107.3912) (width 0.25) (layer B.Cu) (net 2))
 (via (at 144.8308 107.3912) (size 0.6) (drill 0.4) (layers F.Cu B.Cu) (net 2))
 (via (at 152.4508 107.3912) (size 0.6) (drill 0.4) (layers F.Cu B.Cu) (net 2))
 (segment (start 144.8308 107.3912) (end 142.9432 105.5036) (width 0.25) (layer F.Cu) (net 2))
 (segment (start 142.9432 105.5036) (end 141.5011 105.5036) (width 0.25) (layer F.Cu) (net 2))
 (segment (start 155.065 110.0054) (end 152.4508 107.3912) (width 0.25) (layer F.Cu) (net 2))
 (segment (start 155.065 113.2586) (end 155.065 110.0054) (width 0.25) (layer F.Cu) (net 2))
 (segment (start 140.5011 105.5036) (end 141.5011 105.5036) (width 0.25) (layer F.Cu) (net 2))
 (segment (start 144.4244 115.316) (end 143.5011 116.2393) (width 0.25) (layer B.Cu) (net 9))
 (segment (start 143.5011 116.2393) (end 143.5011 117.0036) (width 0.25) (layer B.Cu) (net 9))
 (segment (start 144.4244 112.6998) (end 144.4244 115.316) (width 0.25) (layer B.Cu) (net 9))
 (segment (start 145.796 111.3282) (end 144.4244 112.6998) (width 0.25) (layer B.Cu) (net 9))
 (segment (start 147.3962 111.3282) (end 145.796 111.3282) (width 0.25) (layer B.Cu) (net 9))
 (segment (start 147.955 111.887) (end 147.3962 111.3282) (width 0.25) (layer B.Cu) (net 9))
 (segment (start 148.465 113.2586) (end 148.465 112.397) (width 0.25) (layer F.Cu) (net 9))
 (segment (start 148.465 112.397) (end 147.955 111.887) (width 0.25) (layer F.Cu) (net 9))
 (via (at 147.955 111.887) (size 0.6) (drill 0.4) (layers F.Cu B.Cu) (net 9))
 (segment (start 145.5011 117.0036) (end 145.5011 115.5799) (width 0.25) (layer F.Cu) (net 3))
 (segment (start 152.047807 111.204607) (end 152.865 112.0218) (width 0.25) (layer F.Cu) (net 3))
 (segment (start 145.5011 115.5799) (end 145.034 115.1128) (width 0.25) (layer F.Cu) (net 3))
 (segment (start 145.034 115.1128) (end 145.034 112.0902) (width 0.25) (layer F.Cu) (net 3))
 (segment (start 152.865 112.0218) (end 152.865 113.2586) (width 0.25) (layer F.Cu) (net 3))
 (segment (start 145.034 112.0902) (end 145.919593 111.204607) (width 0.25) (layer F.Cu) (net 3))
 (segment (start 145.919593 111.204607) (end 152.047807 111.204607) (width 0.25) (layer F.Cu) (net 3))
 (segment (start 146.265 114.261) (end 147.5011 115.4971) (width 0.25) (layer F.Cu) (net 7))
 (segment (start 147.5011 115.4971) (end 147.5011 117.0036) (width 0.25) (layer F.Cu) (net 7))
 (segment (start 146.265 113.2586) (end 146.265 114.261) (width 0.25) (layer F.Cu) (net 7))
 (segment (start 149.098 115.5954) (end 149.5011 115.9985) (width 0.25) (layer F.Cu) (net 8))
 (segment (start 149.5011 115.9985) (end 149.5011 117.0036) (width 0.25) (layer F.Cu) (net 8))
 (segment (start 148.463 115.5954) (end 149.098 115.5954) (width 0.25) (layer F.Cu) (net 8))
 (segment (start 147.365 114.4974) (end 148.463 115.5954) (width 0.25) (layer F.Cu) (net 8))
 (segment (start 147.365 113.2586) (end 147.365 114.4974) (width 0.25) (layer F.Cu) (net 8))
 (segment (start 153.4668 114.9858) (end 153.965 114.4876) (width 0.25) (layer F.Cu) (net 4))
 (segment (start 153.965 114.4876) (end 153.965 113.2586) (width 0.25) (layer F.Cu) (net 4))
 (segment (start 152.4 114.9858) (end 153.4668 114.9858) (width 0.25) (layer F.Cu) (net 4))
 (segment (start 151.5011 115.8847) (end 152.4 114.9858) (width 0.25) (layer F.Cu) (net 4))
 (segment (start 151.5011 117.0036) (end 151.5011 115.8847) (width 0.25) (layer F.Cu) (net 4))
 (segment (start 153.5011 115.9599) (end 151.977515 115.9599) (width 0.25) (layer B.Cu) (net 5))
 (segment (start 151.977515 115.9599) (end 150.8252 114.807585) (width 0.25) (layer B.Cu) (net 5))
 (segment (start 150.8252 114.807585) (end 150.8252 114.7826) (width 0.25) (layer B.Cu) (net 5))
 (segment (start 150.8252 114.7826) (end 150.678725 114.636125) (width 0.25) (layer F.Cu) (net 5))
 (segment (start 150.678725 114.636125) (end 150.678725 113.272325) (width 0.25) (layer F.Cu) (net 5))
 (segment (start 150.678725 113.272325) (end 150.665 113.2586) (width 0.25) (layer F.Cu) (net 5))
 (via (at 150.8252 114.7826) (size 0.6) (drill 0.4) (layers F.Cu B.Cu) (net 5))
 (via (at 153.5011 115.9599) (size 0.6) (drill 0.4) (layers F.Cu B.Cu) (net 5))
 (segment (start 153.5011 115.9599) (end 153.5011 117.0036) (width 0.25) (layer F.Cu) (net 5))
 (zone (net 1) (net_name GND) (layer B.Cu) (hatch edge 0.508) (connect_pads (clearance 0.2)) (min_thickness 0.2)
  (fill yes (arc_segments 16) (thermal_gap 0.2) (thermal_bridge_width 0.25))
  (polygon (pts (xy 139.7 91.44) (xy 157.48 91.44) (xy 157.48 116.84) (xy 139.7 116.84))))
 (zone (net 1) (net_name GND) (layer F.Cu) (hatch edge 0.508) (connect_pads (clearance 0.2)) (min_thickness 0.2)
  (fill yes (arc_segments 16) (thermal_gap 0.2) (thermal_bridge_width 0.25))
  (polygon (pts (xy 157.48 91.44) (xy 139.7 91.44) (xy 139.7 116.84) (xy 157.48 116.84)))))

